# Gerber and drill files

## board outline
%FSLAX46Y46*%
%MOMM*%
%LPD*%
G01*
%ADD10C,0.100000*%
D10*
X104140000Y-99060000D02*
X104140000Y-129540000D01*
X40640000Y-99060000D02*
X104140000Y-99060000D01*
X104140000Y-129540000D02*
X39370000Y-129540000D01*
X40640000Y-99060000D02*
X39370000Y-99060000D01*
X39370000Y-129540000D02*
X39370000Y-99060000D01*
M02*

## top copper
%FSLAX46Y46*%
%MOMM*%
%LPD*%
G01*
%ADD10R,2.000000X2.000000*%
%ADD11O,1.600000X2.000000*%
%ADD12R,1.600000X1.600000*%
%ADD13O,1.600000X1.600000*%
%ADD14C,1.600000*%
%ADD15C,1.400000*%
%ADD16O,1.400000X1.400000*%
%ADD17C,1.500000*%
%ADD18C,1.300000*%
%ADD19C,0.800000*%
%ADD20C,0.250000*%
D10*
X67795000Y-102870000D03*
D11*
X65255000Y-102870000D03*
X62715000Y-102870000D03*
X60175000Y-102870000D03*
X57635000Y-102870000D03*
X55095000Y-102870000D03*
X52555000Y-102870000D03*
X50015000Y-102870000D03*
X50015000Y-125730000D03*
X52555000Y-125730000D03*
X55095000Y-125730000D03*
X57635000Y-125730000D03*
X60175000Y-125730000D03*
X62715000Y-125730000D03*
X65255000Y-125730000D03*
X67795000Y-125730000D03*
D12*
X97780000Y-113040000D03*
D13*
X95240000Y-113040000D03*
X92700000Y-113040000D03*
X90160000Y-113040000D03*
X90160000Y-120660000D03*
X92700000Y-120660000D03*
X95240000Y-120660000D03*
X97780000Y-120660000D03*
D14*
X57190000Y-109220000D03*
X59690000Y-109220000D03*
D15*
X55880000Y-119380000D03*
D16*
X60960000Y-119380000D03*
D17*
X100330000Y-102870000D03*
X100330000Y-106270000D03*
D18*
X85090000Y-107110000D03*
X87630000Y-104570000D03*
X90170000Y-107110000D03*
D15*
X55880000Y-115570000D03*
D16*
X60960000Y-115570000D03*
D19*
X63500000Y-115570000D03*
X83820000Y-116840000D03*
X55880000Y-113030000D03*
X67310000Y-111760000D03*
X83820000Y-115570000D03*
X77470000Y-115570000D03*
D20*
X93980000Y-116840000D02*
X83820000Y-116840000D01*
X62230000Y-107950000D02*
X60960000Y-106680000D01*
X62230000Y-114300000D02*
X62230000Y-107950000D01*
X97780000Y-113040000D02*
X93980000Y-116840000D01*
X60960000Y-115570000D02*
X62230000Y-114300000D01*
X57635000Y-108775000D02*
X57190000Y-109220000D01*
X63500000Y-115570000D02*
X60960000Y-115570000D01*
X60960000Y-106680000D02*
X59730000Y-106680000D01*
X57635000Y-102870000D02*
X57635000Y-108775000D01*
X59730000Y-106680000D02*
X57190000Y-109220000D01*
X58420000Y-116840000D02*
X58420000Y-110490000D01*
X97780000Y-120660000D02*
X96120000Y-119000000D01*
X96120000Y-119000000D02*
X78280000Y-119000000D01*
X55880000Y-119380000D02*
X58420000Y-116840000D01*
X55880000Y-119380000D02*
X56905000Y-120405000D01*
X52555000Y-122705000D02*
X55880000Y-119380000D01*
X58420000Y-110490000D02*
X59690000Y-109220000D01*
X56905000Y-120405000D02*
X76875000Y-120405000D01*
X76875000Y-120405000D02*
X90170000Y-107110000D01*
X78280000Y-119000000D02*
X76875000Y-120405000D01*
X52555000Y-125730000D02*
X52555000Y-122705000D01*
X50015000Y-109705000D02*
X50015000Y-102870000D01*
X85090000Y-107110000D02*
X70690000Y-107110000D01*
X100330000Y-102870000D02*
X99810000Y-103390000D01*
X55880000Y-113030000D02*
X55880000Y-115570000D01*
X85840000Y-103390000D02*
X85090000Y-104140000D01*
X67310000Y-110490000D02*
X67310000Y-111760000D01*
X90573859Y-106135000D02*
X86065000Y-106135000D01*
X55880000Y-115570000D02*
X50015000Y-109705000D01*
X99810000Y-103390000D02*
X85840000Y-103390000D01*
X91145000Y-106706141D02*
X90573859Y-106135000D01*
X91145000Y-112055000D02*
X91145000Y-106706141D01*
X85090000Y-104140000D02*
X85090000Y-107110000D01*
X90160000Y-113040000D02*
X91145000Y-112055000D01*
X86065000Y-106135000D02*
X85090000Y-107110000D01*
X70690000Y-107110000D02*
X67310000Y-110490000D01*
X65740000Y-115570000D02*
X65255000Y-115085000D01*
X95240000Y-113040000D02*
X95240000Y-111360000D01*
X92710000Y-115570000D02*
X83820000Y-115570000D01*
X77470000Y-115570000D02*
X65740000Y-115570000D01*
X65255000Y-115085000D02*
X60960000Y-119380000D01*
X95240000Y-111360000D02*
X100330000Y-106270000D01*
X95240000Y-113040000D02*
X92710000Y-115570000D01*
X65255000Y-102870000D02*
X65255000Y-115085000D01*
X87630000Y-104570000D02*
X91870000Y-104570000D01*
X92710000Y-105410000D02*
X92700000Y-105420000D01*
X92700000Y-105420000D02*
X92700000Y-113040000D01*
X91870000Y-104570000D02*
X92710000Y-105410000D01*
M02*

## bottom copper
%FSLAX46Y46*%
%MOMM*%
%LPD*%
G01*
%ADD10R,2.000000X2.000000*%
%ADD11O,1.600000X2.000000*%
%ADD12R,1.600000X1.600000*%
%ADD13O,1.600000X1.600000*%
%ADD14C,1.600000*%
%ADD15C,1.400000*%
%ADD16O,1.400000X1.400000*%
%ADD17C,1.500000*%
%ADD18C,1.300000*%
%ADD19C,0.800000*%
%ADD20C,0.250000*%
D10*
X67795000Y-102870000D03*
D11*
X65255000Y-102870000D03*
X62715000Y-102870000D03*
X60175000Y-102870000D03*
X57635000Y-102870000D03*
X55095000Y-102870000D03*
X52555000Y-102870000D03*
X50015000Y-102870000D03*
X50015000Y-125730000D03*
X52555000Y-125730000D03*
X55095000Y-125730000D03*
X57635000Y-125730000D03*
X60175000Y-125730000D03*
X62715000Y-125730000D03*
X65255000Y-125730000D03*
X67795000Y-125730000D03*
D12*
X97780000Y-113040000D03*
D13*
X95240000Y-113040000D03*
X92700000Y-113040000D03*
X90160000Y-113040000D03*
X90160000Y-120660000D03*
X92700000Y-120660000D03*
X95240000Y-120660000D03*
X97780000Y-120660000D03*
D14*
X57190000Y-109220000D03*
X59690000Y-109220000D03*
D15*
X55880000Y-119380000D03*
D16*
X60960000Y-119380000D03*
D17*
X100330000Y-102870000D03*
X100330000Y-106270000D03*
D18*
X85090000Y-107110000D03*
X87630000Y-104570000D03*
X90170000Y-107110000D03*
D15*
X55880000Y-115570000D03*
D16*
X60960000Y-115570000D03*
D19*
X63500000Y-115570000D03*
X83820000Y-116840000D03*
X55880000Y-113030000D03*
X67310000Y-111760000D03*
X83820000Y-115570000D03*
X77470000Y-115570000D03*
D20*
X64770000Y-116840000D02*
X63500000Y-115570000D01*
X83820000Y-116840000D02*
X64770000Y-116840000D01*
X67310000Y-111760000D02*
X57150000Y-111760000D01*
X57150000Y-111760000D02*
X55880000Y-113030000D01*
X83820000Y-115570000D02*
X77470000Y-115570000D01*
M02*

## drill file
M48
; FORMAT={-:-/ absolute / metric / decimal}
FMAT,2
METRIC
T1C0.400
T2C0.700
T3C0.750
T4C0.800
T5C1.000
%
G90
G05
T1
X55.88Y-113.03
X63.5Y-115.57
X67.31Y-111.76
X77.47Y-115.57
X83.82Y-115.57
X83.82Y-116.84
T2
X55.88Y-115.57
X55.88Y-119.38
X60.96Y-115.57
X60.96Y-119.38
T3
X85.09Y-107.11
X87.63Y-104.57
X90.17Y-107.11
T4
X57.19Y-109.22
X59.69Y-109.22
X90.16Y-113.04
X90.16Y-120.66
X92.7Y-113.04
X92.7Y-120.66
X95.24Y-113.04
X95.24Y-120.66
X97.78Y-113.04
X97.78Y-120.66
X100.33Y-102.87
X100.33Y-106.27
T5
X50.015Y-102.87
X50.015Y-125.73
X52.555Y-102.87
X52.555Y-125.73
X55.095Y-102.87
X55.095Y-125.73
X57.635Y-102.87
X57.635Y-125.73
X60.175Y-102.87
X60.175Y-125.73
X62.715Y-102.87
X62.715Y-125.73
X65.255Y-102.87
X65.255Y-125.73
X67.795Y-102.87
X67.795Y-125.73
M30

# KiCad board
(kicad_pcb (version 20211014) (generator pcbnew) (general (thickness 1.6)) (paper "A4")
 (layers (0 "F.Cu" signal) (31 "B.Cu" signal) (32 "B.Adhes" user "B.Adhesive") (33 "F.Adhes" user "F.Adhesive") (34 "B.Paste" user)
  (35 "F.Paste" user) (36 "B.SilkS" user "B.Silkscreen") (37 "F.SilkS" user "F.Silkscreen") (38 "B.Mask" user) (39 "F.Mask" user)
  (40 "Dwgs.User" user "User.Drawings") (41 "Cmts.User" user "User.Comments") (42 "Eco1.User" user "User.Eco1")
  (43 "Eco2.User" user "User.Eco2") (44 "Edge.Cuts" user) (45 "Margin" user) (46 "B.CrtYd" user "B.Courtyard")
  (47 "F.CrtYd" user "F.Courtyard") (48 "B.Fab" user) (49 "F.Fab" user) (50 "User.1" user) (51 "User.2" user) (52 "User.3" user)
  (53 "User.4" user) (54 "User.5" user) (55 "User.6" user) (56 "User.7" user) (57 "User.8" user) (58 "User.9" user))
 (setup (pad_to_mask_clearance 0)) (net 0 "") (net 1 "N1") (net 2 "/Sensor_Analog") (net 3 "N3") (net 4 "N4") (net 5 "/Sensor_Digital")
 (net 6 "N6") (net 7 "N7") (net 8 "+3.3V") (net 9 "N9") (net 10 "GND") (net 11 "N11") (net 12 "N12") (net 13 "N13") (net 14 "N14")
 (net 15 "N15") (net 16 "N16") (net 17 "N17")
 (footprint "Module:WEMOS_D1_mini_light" (layer "F.Cu") (at 67.795 102.87 -90)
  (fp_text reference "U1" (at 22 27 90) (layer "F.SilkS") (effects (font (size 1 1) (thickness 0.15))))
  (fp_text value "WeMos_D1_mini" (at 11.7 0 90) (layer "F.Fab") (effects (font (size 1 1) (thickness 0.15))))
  (pad "1" thru_hole rect (at 0 0 270) (size 2 2) (drill 1) (layers *.Cu *.Mask) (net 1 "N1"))
  (pad "2" thru_hole oval (at 0 2.54 270) (size 2 1.6) (drill 1) (layers *.Cu *.Mask) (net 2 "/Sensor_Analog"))
  (pad "3" thru_hole oval (at 0 5.08 270) (size 2 1.6) (drill 1) (layers *.Cu *.Mask) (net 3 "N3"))
  (pad "4" thru_hole oval (at 0 7.62 270) (size 2 1.6) (drill 1) (layers *.Cu *.Mask) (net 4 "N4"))
  (pad "5" thru_hole oval (at 0 10.16 270) (size 2 1.6) (drill 1) (layers *.Cu *.Mask) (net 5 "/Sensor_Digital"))
  (pad "6" thru_hole oval (at 0 12.7 270) (size 2 1.6) (drill 1) (layers *.Cu *.Mask) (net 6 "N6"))
  (pad "7" thru_hole oval (at 0 15.24 270) (size 2 1.6) (drill 1) (layers *.Cu *.Mask) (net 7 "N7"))
  (pad "8" thru_hole oval (at 0 17.78 270) (size 2 1.6) (drill 1) (layers *.Cu *.Mask) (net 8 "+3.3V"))
  (pad "9" thru_hole oval (at 22.86 17.78 270) (size 2 1.6) (drill 1) (layers *.Cu *.Mask) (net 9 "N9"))
  (pad "10" thru_hole oval (at 22.86 15.24 270) (size 2 1.6) (drill 1) (layers *.Cu *.Mask) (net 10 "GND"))
  (pad "11" thru_hole oval (at 22.86 12.7 270) (size 2 1.6) (drill 1) (layers *.Cu *.Mask) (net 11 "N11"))
  (pad "12" thru_hole oval (at 22.86 10.16 270) (size 2 1.6) (drill 1) (layers *.Cu *.Mask) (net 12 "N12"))
  (pad "13" thru_hole oval (at 22.86 7.62 270) (size 2 1.6) (drill 1) (layers *.Cu *.Mask) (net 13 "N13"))
  (pad "14" thru_hole oval (at 22.86 5.08 270) (size 2 1.6) (drill 1) (layers *.Cu *.Mask) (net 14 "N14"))
  (pad "15" thru_hole oval (at 22.86 2.54 270) (size 2 1.6) (drill 1) (layers *.Cu *.Mask) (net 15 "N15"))
  (pad "16" thru_hole oval (at 22.86 0 270) (size 2 1.6) (drill 1) (layers *.Cu *.Mask) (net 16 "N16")))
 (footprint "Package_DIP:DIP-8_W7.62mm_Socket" (layer "F.Cu") (at 97.78 113.04 -90)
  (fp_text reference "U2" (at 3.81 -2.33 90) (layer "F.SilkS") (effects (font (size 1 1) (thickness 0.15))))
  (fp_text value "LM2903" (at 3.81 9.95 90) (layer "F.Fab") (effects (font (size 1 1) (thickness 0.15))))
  (pad "1" thru_hole rect (at 0 0 270) (size 1.6 1.6) (drill 0.8) (layers *.Cu *.Mask) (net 5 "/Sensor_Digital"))
  (pad "2" thru_hole oval (at 0 2.54 270) (size 1.6 1.6) (drill 0.8) (layers *.Cu *.Mask) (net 2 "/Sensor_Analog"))
  (pad "3" thru_hole oval (at 0 5.08 270) (size 1.6 1.6) (drill 0.8) (layers *.Cu *.Mask) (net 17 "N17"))
  (pad "4" thru_hole oval (at 0 7.62 270) (size 1.6 1.6) (drill 0.8) (layers *.Cu *.Mask) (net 8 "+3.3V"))
  (pad "5" thru_hole oval (at 7.62 7.62 270) (size 1.6 1.6) (drill 0.8) (layers *.Cu *.Mask))
  (pad "6" thru_hole oval (at 7.62 5.08 270) (size 1.6 1.6) (drill 0.8) (layers *.Cu *.Mask))
  (pad "7" thru_hole oval (at 7.62 2.54 270) (size 1.6 1.6) (drill 0.8) (layers *.Cu *.Mask))
  (pad "8" thru_hole oval (at 7.62 0 270) (size 1.6 1.6) (drill 0.8) (layers *.Cu *.Mask) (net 10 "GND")))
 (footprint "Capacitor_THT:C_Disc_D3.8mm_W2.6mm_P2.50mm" (layer "F.Cu") (at 57.19 109.22)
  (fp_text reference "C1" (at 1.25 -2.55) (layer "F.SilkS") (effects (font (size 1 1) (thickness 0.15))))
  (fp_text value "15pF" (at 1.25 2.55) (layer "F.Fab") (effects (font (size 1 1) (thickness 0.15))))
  (pad "1" thru_hole circle (at 0 0) (size 1.6 1.6) (drill 0.8) (layers *.Cu *.Mask) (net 5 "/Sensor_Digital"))
  (pad "2" thru_hole circle (at 2.5 0) (size 1.6 1.6) (drill 0.8) (layers *.Cu *.Mask) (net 10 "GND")))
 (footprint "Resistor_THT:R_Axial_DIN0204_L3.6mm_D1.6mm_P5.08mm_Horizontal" (layer "F.Cu") (at 55.88 119.38)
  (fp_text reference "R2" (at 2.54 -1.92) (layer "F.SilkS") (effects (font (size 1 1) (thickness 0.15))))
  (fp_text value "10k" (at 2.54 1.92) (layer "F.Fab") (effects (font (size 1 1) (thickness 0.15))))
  (pad "1" thru_hole circle (at 0 0) (size 1.4 1.4) (drill 0.7) (layers *.Cu *.Mask) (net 10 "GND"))
  (pad "2" thru_hole oval (at 5.08 0) (size 1.4 1.4) (drill 0.7) (layers *.Cu *.Mask) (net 2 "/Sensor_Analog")))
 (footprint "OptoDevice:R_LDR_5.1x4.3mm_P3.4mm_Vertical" (layer "F.Cu") (at 100.33 102.87 -90)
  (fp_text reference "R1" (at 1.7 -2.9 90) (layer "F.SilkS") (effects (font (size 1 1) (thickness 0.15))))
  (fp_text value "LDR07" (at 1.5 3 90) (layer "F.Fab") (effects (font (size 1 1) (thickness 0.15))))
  (pad "1" thru_hole circle (at 0 0 270) (size 1.5 1.5) (drill 0.8) (layers *.Cu *.Mask) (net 8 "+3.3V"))
  (pad "2" thru_hole circle (at 3.4 0 270) (size 1.5 1.5) (drill 0.8) (layers *.Cu *.Mask) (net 2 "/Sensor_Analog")))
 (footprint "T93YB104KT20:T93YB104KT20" (layer "F.Cu") (at 85.09 107.11)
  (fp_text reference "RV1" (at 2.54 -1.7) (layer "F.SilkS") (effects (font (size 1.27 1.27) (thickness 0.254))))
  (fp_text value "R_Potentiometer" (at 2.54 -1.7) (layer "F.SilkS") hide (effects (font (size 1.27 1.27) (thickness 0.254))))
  (pad "1" thru_hole circle locked (at 0 0) (size 1.3 1.3) (drill 0.75) (layers *.Cu *.Mask) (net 8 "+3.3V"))
  (pad "2" thru_hole circle locked (at 2.54 -2.54) (size 1.3 1.3) (drill 0.75) (layers *.Cu *.Mask) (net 17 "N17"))
  (pad "3" thru_hole circle locked (at 5.08 0) (size 1.3 1.3) (drill 0.75) (layers *.Cu *.Mask) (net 10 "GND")))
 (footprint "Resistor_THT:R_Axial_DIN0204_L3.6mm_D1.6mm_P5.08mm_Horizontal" (layer "F.Cu") (at 55.88 115.57)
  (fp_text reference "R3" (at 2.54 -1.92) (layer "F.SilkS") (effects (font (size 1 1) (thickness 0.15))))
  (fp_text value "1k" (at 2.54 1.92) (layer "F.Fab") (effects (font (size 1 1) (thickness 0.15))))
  (pad "1" thru_hole circle (at 0 0) (size 1.4 1.4) (drill 0.7) (layers *.Cu *.Mask) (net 8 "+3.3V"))
  (pad "2" thru_hole oval (at 5.08 0) (size 1.4 1.4) (drill 0.7) (layers *.Cu *.Mask) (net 5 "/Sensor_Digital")))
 (gr_line (start 104.14 99.06) (end 104.14 129.54) (layer "Edge.Cuts") (width 0.1))
 (gr_line (start 40.64 99.06) (end 104.14 99.06) (layer "Edge.Cuts") (width 0.1))
 (gr_line (start 104.14 129.54) (end 39.37 129.54) (layer "Edge.Cuts") (width 0.1))
 (gr_line (start 40.64 99.06) (end 39.37 99.06) (layer "Edge.Cuts") (width 0.1))
 (gr_line (start 39.37 129.54) (end 39.37 99.06) (layer "Edge.Cuts") (width 0.1))
 (segment (start 93.98 116.84) (end 83.82 116.84) (width 0.25) (layer "F.Cu") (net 5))
 (segment (start 62.23 107.95) (end 60.96 106.68) (width 0.25) (layer "F.Cu") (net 5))
 (segment (start 62.23 114.3) (end 62.23 107.95) (width 0.25) (layer "F.Cu") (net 5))
 (segment (start 97.78 113.04) (end 93.98 116.84) (width 0.25) (layer "F.Cu") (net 5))
 (segment (start 60.96 115.57) (end 62.23 114.3) (width 0.25) (layer "F.Cu") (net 5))
 (segment (start 57.635 108.775) (end 57.19 109.22) (width 0.25) (layer "F.Cu") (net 5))
 (segment (start 63.5 115.57) (end 60.96 115.57) (width 0.25) (layer "F.Cu") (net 5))
 (segment (start 60.96 106.68) (end 59.73 106.68) (width 0.25) (layer "F.Cu") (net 5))
 (segment (start 57.635 102.87) (end 57.635 108.775) (width 0.25) (layer "F.Cu") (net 5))
 (segment (start 59.73 106.68) (end 57.19 109.22) (width 0.25) (layer "F.Cu") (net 5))
 (via (at 63.5 115.57) (size 0.8) (drill 0.4) (layers "F.Cu" "B.Cu") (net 5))
 (via (at 83.82 116.84) (size 0.8) (drill 0.4) (layers "F.Cu" "B.Cu") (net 5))
 (segment (start 64.77 116.84) (end 63.5 115.57) (width 0.25) (layer "B.Cu") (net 5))
 (segment (start 83.82 116.84) (end 64.77 116.84) (width 0.25) (layer "B.Cu") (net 5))
 (segment (start 58.42 116.84) (end 58.42 110.49) (width 0.25) (layer "F.Cu") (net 10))
 (segment (start 97.78 120.66) (end 96.12 119) (width 0.25) (layer "F.Cu") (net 10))
 (segment (start 96.12 119) (end 78.28 119) (width 0.25) (layer "F.Cu") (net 10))
 (segment (start 55.88 119.38) (end 58.42 116.84) (width 0.25) (layer "F.Cu") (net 10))
 (segment (start 55.88 119.38) (end 56.905 120.405) (width 0.25) (layer "F.Cu") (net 10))
 (segment (start 52.555 122.705) (end 55.88 119.38) (width 0.25) (layer "F.Cu") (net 10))
 (segment (start 58.42 110.49) (end 59.69 109.22) (width 0.25) (layer "F.Cu") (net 10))
 (segment (start 56.905 120.405) (end 76.875 120.405) (width 0.25) (layer "F.Cu") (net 10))
 (segment (start 76.875 120.405) (end 90.17 107.11) (width 0.25) (layer "F.Cu") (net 10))
 (segment (start 78.28 119) (end 76.875 120.405) (width 0.25) (layer "F.Cu") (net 10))
 (segment (start 52.555 125.73) (end 52.555 122.705) (width 0.25) (layer "F.Cu") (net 10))
 (segment (start 50.015 109.705) (end 50.015 102.87) (width 0.25) (layer "F.Cu") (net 8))
 (segment (start 85.09 107.11) (end 70.69 107.11) (width 0.25) (layer "F.Cu") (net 8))
 (segment (start 100.33 102.87) (end 99.81 103.39) (width 0.25) (layer "F.Cu") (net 8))
 (segment (start 55.88 113.03) (end 55.88 115.57) (width 0.25) (layer "F.Cu") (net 8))
 (segment (start 85.84 103.39) (end 85.09 104.14) (width 0.25) (layer "F.Cu") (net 8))
 (segment (start 67.31 110.49) (end 67.31 111.76) (width 0.25) (layer "F.Cu") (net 8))
 (segment (start 90.573859 106.135) (end 86.065 106.135) (width 0.25) (layer "F.Cu") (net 8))
 (segment (start 55.88 115.57) (end 50.015 109.705) (width 0.25) (layer "F.Cu") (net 8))
 (segment (start 99.81 103.39) (end 85.84 103.39) (width 0.25) (layer "F.Cu") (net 8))
 (segment (start 91.145 106.706141) (end 90.573859 106.135) (width 0.25) (layer "F.Cu") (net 8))
 (segment (start 91.145 112.055) (end 91.145 106.706141) (width 0.25) (layer "F.Cu") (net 8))
 (segment (start 85.09 104.14) (end 85.09 107.11) (width 0.25) (layer "F.Cu") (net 8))
 (segment (start 90.16 113.04) (end 91.145 112.055) (width 0.25) (layer "F.Cu") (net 8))
 (segment (start 86.065 106.135) (end 85.09 107.11) (width 0.25) (layer "F.Cu") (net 8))
 (segment (start 70.69 107.11) (end 67.31 110.49) (width 0.25) (layer "F.Cu") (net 8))
 (via (at 55.88 113.03) (size 0.8) (drill 0.4) (layers "F.Cu" "B.Cu") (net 8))
 (via (at 67.31 111.76) (size 0.8) (drill 0.4) (layers "F.Cu" "B.Cu") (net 8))
 (segment (start 67.31 111.76) (end 57.15 111.76) (width 0.25) (layer "B.Cu") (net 8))
 (segment (start 57.15 111.76) (end 55.88 113.03) (width 0.25) (layer "B.Cu") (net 8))
 (segment (start 65.74 115.57) (end 65.255 115.085) (width 0.25) (layer "F.Cu") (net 2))
 (segment (start 95.24 113.04) (end 95.24 111.36) (width 0.25) (layer "F.Cu") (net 2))
 (segment (start 92.71 115.57) (end 83.82 115.57) (width 0.25) (layer "F.Cu") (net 2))
 (segment (start 77.47 115.57) (end 65.74 115.57) (width 0.25) (layer "F.Cu") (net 2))
 (segment (start 65.255 115.085) (end 60.96 119.38) (width 0.25) (layer "F.Cu") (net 2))
 (segment (start 95.24 111.36) (end 100.33 106.27) (width 0.25) (layer "F.Cu") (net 2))
 (segment (start 95.24 113.04) (end 92.71 115.57) (width 0.25) (layer "F.Cu") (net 2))
 (segment (start 65.255 102.87) (end 65.255 115.085) (width 0.25) (layer "F.Cu") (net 2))
 (via (at 83.82 115.57) (size 0.8) (drill 0.4) (layers "F.Cu" "B.Cu") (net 2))
 (via (at 77.47 115.57) (size 0.8) (drill 0.4) (layers "F.Cu" "B.Cu") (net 2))
 (segment (start 83.82 115.57) (end 77.47 115.57) (width 0.25) (layer "B.Cu") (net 2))
 (segment (start 87.63 104.57) (end 91.87 104.57) (width 0.25) (layer "F.Cu") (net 17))
 (segment (start 92.71 105.41) (end 92.7 105.42) (width 0.25) (layer "F.Cu") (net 17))
 (segment (start 92.7 105.42) (end 92.7 113.04) (width 0.25) (layer "F.Cu") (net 17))
 (segment (start 91.87 104.57) (end 92.71 105.41) (width 0.25) (layer "F.Cu") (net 17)))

